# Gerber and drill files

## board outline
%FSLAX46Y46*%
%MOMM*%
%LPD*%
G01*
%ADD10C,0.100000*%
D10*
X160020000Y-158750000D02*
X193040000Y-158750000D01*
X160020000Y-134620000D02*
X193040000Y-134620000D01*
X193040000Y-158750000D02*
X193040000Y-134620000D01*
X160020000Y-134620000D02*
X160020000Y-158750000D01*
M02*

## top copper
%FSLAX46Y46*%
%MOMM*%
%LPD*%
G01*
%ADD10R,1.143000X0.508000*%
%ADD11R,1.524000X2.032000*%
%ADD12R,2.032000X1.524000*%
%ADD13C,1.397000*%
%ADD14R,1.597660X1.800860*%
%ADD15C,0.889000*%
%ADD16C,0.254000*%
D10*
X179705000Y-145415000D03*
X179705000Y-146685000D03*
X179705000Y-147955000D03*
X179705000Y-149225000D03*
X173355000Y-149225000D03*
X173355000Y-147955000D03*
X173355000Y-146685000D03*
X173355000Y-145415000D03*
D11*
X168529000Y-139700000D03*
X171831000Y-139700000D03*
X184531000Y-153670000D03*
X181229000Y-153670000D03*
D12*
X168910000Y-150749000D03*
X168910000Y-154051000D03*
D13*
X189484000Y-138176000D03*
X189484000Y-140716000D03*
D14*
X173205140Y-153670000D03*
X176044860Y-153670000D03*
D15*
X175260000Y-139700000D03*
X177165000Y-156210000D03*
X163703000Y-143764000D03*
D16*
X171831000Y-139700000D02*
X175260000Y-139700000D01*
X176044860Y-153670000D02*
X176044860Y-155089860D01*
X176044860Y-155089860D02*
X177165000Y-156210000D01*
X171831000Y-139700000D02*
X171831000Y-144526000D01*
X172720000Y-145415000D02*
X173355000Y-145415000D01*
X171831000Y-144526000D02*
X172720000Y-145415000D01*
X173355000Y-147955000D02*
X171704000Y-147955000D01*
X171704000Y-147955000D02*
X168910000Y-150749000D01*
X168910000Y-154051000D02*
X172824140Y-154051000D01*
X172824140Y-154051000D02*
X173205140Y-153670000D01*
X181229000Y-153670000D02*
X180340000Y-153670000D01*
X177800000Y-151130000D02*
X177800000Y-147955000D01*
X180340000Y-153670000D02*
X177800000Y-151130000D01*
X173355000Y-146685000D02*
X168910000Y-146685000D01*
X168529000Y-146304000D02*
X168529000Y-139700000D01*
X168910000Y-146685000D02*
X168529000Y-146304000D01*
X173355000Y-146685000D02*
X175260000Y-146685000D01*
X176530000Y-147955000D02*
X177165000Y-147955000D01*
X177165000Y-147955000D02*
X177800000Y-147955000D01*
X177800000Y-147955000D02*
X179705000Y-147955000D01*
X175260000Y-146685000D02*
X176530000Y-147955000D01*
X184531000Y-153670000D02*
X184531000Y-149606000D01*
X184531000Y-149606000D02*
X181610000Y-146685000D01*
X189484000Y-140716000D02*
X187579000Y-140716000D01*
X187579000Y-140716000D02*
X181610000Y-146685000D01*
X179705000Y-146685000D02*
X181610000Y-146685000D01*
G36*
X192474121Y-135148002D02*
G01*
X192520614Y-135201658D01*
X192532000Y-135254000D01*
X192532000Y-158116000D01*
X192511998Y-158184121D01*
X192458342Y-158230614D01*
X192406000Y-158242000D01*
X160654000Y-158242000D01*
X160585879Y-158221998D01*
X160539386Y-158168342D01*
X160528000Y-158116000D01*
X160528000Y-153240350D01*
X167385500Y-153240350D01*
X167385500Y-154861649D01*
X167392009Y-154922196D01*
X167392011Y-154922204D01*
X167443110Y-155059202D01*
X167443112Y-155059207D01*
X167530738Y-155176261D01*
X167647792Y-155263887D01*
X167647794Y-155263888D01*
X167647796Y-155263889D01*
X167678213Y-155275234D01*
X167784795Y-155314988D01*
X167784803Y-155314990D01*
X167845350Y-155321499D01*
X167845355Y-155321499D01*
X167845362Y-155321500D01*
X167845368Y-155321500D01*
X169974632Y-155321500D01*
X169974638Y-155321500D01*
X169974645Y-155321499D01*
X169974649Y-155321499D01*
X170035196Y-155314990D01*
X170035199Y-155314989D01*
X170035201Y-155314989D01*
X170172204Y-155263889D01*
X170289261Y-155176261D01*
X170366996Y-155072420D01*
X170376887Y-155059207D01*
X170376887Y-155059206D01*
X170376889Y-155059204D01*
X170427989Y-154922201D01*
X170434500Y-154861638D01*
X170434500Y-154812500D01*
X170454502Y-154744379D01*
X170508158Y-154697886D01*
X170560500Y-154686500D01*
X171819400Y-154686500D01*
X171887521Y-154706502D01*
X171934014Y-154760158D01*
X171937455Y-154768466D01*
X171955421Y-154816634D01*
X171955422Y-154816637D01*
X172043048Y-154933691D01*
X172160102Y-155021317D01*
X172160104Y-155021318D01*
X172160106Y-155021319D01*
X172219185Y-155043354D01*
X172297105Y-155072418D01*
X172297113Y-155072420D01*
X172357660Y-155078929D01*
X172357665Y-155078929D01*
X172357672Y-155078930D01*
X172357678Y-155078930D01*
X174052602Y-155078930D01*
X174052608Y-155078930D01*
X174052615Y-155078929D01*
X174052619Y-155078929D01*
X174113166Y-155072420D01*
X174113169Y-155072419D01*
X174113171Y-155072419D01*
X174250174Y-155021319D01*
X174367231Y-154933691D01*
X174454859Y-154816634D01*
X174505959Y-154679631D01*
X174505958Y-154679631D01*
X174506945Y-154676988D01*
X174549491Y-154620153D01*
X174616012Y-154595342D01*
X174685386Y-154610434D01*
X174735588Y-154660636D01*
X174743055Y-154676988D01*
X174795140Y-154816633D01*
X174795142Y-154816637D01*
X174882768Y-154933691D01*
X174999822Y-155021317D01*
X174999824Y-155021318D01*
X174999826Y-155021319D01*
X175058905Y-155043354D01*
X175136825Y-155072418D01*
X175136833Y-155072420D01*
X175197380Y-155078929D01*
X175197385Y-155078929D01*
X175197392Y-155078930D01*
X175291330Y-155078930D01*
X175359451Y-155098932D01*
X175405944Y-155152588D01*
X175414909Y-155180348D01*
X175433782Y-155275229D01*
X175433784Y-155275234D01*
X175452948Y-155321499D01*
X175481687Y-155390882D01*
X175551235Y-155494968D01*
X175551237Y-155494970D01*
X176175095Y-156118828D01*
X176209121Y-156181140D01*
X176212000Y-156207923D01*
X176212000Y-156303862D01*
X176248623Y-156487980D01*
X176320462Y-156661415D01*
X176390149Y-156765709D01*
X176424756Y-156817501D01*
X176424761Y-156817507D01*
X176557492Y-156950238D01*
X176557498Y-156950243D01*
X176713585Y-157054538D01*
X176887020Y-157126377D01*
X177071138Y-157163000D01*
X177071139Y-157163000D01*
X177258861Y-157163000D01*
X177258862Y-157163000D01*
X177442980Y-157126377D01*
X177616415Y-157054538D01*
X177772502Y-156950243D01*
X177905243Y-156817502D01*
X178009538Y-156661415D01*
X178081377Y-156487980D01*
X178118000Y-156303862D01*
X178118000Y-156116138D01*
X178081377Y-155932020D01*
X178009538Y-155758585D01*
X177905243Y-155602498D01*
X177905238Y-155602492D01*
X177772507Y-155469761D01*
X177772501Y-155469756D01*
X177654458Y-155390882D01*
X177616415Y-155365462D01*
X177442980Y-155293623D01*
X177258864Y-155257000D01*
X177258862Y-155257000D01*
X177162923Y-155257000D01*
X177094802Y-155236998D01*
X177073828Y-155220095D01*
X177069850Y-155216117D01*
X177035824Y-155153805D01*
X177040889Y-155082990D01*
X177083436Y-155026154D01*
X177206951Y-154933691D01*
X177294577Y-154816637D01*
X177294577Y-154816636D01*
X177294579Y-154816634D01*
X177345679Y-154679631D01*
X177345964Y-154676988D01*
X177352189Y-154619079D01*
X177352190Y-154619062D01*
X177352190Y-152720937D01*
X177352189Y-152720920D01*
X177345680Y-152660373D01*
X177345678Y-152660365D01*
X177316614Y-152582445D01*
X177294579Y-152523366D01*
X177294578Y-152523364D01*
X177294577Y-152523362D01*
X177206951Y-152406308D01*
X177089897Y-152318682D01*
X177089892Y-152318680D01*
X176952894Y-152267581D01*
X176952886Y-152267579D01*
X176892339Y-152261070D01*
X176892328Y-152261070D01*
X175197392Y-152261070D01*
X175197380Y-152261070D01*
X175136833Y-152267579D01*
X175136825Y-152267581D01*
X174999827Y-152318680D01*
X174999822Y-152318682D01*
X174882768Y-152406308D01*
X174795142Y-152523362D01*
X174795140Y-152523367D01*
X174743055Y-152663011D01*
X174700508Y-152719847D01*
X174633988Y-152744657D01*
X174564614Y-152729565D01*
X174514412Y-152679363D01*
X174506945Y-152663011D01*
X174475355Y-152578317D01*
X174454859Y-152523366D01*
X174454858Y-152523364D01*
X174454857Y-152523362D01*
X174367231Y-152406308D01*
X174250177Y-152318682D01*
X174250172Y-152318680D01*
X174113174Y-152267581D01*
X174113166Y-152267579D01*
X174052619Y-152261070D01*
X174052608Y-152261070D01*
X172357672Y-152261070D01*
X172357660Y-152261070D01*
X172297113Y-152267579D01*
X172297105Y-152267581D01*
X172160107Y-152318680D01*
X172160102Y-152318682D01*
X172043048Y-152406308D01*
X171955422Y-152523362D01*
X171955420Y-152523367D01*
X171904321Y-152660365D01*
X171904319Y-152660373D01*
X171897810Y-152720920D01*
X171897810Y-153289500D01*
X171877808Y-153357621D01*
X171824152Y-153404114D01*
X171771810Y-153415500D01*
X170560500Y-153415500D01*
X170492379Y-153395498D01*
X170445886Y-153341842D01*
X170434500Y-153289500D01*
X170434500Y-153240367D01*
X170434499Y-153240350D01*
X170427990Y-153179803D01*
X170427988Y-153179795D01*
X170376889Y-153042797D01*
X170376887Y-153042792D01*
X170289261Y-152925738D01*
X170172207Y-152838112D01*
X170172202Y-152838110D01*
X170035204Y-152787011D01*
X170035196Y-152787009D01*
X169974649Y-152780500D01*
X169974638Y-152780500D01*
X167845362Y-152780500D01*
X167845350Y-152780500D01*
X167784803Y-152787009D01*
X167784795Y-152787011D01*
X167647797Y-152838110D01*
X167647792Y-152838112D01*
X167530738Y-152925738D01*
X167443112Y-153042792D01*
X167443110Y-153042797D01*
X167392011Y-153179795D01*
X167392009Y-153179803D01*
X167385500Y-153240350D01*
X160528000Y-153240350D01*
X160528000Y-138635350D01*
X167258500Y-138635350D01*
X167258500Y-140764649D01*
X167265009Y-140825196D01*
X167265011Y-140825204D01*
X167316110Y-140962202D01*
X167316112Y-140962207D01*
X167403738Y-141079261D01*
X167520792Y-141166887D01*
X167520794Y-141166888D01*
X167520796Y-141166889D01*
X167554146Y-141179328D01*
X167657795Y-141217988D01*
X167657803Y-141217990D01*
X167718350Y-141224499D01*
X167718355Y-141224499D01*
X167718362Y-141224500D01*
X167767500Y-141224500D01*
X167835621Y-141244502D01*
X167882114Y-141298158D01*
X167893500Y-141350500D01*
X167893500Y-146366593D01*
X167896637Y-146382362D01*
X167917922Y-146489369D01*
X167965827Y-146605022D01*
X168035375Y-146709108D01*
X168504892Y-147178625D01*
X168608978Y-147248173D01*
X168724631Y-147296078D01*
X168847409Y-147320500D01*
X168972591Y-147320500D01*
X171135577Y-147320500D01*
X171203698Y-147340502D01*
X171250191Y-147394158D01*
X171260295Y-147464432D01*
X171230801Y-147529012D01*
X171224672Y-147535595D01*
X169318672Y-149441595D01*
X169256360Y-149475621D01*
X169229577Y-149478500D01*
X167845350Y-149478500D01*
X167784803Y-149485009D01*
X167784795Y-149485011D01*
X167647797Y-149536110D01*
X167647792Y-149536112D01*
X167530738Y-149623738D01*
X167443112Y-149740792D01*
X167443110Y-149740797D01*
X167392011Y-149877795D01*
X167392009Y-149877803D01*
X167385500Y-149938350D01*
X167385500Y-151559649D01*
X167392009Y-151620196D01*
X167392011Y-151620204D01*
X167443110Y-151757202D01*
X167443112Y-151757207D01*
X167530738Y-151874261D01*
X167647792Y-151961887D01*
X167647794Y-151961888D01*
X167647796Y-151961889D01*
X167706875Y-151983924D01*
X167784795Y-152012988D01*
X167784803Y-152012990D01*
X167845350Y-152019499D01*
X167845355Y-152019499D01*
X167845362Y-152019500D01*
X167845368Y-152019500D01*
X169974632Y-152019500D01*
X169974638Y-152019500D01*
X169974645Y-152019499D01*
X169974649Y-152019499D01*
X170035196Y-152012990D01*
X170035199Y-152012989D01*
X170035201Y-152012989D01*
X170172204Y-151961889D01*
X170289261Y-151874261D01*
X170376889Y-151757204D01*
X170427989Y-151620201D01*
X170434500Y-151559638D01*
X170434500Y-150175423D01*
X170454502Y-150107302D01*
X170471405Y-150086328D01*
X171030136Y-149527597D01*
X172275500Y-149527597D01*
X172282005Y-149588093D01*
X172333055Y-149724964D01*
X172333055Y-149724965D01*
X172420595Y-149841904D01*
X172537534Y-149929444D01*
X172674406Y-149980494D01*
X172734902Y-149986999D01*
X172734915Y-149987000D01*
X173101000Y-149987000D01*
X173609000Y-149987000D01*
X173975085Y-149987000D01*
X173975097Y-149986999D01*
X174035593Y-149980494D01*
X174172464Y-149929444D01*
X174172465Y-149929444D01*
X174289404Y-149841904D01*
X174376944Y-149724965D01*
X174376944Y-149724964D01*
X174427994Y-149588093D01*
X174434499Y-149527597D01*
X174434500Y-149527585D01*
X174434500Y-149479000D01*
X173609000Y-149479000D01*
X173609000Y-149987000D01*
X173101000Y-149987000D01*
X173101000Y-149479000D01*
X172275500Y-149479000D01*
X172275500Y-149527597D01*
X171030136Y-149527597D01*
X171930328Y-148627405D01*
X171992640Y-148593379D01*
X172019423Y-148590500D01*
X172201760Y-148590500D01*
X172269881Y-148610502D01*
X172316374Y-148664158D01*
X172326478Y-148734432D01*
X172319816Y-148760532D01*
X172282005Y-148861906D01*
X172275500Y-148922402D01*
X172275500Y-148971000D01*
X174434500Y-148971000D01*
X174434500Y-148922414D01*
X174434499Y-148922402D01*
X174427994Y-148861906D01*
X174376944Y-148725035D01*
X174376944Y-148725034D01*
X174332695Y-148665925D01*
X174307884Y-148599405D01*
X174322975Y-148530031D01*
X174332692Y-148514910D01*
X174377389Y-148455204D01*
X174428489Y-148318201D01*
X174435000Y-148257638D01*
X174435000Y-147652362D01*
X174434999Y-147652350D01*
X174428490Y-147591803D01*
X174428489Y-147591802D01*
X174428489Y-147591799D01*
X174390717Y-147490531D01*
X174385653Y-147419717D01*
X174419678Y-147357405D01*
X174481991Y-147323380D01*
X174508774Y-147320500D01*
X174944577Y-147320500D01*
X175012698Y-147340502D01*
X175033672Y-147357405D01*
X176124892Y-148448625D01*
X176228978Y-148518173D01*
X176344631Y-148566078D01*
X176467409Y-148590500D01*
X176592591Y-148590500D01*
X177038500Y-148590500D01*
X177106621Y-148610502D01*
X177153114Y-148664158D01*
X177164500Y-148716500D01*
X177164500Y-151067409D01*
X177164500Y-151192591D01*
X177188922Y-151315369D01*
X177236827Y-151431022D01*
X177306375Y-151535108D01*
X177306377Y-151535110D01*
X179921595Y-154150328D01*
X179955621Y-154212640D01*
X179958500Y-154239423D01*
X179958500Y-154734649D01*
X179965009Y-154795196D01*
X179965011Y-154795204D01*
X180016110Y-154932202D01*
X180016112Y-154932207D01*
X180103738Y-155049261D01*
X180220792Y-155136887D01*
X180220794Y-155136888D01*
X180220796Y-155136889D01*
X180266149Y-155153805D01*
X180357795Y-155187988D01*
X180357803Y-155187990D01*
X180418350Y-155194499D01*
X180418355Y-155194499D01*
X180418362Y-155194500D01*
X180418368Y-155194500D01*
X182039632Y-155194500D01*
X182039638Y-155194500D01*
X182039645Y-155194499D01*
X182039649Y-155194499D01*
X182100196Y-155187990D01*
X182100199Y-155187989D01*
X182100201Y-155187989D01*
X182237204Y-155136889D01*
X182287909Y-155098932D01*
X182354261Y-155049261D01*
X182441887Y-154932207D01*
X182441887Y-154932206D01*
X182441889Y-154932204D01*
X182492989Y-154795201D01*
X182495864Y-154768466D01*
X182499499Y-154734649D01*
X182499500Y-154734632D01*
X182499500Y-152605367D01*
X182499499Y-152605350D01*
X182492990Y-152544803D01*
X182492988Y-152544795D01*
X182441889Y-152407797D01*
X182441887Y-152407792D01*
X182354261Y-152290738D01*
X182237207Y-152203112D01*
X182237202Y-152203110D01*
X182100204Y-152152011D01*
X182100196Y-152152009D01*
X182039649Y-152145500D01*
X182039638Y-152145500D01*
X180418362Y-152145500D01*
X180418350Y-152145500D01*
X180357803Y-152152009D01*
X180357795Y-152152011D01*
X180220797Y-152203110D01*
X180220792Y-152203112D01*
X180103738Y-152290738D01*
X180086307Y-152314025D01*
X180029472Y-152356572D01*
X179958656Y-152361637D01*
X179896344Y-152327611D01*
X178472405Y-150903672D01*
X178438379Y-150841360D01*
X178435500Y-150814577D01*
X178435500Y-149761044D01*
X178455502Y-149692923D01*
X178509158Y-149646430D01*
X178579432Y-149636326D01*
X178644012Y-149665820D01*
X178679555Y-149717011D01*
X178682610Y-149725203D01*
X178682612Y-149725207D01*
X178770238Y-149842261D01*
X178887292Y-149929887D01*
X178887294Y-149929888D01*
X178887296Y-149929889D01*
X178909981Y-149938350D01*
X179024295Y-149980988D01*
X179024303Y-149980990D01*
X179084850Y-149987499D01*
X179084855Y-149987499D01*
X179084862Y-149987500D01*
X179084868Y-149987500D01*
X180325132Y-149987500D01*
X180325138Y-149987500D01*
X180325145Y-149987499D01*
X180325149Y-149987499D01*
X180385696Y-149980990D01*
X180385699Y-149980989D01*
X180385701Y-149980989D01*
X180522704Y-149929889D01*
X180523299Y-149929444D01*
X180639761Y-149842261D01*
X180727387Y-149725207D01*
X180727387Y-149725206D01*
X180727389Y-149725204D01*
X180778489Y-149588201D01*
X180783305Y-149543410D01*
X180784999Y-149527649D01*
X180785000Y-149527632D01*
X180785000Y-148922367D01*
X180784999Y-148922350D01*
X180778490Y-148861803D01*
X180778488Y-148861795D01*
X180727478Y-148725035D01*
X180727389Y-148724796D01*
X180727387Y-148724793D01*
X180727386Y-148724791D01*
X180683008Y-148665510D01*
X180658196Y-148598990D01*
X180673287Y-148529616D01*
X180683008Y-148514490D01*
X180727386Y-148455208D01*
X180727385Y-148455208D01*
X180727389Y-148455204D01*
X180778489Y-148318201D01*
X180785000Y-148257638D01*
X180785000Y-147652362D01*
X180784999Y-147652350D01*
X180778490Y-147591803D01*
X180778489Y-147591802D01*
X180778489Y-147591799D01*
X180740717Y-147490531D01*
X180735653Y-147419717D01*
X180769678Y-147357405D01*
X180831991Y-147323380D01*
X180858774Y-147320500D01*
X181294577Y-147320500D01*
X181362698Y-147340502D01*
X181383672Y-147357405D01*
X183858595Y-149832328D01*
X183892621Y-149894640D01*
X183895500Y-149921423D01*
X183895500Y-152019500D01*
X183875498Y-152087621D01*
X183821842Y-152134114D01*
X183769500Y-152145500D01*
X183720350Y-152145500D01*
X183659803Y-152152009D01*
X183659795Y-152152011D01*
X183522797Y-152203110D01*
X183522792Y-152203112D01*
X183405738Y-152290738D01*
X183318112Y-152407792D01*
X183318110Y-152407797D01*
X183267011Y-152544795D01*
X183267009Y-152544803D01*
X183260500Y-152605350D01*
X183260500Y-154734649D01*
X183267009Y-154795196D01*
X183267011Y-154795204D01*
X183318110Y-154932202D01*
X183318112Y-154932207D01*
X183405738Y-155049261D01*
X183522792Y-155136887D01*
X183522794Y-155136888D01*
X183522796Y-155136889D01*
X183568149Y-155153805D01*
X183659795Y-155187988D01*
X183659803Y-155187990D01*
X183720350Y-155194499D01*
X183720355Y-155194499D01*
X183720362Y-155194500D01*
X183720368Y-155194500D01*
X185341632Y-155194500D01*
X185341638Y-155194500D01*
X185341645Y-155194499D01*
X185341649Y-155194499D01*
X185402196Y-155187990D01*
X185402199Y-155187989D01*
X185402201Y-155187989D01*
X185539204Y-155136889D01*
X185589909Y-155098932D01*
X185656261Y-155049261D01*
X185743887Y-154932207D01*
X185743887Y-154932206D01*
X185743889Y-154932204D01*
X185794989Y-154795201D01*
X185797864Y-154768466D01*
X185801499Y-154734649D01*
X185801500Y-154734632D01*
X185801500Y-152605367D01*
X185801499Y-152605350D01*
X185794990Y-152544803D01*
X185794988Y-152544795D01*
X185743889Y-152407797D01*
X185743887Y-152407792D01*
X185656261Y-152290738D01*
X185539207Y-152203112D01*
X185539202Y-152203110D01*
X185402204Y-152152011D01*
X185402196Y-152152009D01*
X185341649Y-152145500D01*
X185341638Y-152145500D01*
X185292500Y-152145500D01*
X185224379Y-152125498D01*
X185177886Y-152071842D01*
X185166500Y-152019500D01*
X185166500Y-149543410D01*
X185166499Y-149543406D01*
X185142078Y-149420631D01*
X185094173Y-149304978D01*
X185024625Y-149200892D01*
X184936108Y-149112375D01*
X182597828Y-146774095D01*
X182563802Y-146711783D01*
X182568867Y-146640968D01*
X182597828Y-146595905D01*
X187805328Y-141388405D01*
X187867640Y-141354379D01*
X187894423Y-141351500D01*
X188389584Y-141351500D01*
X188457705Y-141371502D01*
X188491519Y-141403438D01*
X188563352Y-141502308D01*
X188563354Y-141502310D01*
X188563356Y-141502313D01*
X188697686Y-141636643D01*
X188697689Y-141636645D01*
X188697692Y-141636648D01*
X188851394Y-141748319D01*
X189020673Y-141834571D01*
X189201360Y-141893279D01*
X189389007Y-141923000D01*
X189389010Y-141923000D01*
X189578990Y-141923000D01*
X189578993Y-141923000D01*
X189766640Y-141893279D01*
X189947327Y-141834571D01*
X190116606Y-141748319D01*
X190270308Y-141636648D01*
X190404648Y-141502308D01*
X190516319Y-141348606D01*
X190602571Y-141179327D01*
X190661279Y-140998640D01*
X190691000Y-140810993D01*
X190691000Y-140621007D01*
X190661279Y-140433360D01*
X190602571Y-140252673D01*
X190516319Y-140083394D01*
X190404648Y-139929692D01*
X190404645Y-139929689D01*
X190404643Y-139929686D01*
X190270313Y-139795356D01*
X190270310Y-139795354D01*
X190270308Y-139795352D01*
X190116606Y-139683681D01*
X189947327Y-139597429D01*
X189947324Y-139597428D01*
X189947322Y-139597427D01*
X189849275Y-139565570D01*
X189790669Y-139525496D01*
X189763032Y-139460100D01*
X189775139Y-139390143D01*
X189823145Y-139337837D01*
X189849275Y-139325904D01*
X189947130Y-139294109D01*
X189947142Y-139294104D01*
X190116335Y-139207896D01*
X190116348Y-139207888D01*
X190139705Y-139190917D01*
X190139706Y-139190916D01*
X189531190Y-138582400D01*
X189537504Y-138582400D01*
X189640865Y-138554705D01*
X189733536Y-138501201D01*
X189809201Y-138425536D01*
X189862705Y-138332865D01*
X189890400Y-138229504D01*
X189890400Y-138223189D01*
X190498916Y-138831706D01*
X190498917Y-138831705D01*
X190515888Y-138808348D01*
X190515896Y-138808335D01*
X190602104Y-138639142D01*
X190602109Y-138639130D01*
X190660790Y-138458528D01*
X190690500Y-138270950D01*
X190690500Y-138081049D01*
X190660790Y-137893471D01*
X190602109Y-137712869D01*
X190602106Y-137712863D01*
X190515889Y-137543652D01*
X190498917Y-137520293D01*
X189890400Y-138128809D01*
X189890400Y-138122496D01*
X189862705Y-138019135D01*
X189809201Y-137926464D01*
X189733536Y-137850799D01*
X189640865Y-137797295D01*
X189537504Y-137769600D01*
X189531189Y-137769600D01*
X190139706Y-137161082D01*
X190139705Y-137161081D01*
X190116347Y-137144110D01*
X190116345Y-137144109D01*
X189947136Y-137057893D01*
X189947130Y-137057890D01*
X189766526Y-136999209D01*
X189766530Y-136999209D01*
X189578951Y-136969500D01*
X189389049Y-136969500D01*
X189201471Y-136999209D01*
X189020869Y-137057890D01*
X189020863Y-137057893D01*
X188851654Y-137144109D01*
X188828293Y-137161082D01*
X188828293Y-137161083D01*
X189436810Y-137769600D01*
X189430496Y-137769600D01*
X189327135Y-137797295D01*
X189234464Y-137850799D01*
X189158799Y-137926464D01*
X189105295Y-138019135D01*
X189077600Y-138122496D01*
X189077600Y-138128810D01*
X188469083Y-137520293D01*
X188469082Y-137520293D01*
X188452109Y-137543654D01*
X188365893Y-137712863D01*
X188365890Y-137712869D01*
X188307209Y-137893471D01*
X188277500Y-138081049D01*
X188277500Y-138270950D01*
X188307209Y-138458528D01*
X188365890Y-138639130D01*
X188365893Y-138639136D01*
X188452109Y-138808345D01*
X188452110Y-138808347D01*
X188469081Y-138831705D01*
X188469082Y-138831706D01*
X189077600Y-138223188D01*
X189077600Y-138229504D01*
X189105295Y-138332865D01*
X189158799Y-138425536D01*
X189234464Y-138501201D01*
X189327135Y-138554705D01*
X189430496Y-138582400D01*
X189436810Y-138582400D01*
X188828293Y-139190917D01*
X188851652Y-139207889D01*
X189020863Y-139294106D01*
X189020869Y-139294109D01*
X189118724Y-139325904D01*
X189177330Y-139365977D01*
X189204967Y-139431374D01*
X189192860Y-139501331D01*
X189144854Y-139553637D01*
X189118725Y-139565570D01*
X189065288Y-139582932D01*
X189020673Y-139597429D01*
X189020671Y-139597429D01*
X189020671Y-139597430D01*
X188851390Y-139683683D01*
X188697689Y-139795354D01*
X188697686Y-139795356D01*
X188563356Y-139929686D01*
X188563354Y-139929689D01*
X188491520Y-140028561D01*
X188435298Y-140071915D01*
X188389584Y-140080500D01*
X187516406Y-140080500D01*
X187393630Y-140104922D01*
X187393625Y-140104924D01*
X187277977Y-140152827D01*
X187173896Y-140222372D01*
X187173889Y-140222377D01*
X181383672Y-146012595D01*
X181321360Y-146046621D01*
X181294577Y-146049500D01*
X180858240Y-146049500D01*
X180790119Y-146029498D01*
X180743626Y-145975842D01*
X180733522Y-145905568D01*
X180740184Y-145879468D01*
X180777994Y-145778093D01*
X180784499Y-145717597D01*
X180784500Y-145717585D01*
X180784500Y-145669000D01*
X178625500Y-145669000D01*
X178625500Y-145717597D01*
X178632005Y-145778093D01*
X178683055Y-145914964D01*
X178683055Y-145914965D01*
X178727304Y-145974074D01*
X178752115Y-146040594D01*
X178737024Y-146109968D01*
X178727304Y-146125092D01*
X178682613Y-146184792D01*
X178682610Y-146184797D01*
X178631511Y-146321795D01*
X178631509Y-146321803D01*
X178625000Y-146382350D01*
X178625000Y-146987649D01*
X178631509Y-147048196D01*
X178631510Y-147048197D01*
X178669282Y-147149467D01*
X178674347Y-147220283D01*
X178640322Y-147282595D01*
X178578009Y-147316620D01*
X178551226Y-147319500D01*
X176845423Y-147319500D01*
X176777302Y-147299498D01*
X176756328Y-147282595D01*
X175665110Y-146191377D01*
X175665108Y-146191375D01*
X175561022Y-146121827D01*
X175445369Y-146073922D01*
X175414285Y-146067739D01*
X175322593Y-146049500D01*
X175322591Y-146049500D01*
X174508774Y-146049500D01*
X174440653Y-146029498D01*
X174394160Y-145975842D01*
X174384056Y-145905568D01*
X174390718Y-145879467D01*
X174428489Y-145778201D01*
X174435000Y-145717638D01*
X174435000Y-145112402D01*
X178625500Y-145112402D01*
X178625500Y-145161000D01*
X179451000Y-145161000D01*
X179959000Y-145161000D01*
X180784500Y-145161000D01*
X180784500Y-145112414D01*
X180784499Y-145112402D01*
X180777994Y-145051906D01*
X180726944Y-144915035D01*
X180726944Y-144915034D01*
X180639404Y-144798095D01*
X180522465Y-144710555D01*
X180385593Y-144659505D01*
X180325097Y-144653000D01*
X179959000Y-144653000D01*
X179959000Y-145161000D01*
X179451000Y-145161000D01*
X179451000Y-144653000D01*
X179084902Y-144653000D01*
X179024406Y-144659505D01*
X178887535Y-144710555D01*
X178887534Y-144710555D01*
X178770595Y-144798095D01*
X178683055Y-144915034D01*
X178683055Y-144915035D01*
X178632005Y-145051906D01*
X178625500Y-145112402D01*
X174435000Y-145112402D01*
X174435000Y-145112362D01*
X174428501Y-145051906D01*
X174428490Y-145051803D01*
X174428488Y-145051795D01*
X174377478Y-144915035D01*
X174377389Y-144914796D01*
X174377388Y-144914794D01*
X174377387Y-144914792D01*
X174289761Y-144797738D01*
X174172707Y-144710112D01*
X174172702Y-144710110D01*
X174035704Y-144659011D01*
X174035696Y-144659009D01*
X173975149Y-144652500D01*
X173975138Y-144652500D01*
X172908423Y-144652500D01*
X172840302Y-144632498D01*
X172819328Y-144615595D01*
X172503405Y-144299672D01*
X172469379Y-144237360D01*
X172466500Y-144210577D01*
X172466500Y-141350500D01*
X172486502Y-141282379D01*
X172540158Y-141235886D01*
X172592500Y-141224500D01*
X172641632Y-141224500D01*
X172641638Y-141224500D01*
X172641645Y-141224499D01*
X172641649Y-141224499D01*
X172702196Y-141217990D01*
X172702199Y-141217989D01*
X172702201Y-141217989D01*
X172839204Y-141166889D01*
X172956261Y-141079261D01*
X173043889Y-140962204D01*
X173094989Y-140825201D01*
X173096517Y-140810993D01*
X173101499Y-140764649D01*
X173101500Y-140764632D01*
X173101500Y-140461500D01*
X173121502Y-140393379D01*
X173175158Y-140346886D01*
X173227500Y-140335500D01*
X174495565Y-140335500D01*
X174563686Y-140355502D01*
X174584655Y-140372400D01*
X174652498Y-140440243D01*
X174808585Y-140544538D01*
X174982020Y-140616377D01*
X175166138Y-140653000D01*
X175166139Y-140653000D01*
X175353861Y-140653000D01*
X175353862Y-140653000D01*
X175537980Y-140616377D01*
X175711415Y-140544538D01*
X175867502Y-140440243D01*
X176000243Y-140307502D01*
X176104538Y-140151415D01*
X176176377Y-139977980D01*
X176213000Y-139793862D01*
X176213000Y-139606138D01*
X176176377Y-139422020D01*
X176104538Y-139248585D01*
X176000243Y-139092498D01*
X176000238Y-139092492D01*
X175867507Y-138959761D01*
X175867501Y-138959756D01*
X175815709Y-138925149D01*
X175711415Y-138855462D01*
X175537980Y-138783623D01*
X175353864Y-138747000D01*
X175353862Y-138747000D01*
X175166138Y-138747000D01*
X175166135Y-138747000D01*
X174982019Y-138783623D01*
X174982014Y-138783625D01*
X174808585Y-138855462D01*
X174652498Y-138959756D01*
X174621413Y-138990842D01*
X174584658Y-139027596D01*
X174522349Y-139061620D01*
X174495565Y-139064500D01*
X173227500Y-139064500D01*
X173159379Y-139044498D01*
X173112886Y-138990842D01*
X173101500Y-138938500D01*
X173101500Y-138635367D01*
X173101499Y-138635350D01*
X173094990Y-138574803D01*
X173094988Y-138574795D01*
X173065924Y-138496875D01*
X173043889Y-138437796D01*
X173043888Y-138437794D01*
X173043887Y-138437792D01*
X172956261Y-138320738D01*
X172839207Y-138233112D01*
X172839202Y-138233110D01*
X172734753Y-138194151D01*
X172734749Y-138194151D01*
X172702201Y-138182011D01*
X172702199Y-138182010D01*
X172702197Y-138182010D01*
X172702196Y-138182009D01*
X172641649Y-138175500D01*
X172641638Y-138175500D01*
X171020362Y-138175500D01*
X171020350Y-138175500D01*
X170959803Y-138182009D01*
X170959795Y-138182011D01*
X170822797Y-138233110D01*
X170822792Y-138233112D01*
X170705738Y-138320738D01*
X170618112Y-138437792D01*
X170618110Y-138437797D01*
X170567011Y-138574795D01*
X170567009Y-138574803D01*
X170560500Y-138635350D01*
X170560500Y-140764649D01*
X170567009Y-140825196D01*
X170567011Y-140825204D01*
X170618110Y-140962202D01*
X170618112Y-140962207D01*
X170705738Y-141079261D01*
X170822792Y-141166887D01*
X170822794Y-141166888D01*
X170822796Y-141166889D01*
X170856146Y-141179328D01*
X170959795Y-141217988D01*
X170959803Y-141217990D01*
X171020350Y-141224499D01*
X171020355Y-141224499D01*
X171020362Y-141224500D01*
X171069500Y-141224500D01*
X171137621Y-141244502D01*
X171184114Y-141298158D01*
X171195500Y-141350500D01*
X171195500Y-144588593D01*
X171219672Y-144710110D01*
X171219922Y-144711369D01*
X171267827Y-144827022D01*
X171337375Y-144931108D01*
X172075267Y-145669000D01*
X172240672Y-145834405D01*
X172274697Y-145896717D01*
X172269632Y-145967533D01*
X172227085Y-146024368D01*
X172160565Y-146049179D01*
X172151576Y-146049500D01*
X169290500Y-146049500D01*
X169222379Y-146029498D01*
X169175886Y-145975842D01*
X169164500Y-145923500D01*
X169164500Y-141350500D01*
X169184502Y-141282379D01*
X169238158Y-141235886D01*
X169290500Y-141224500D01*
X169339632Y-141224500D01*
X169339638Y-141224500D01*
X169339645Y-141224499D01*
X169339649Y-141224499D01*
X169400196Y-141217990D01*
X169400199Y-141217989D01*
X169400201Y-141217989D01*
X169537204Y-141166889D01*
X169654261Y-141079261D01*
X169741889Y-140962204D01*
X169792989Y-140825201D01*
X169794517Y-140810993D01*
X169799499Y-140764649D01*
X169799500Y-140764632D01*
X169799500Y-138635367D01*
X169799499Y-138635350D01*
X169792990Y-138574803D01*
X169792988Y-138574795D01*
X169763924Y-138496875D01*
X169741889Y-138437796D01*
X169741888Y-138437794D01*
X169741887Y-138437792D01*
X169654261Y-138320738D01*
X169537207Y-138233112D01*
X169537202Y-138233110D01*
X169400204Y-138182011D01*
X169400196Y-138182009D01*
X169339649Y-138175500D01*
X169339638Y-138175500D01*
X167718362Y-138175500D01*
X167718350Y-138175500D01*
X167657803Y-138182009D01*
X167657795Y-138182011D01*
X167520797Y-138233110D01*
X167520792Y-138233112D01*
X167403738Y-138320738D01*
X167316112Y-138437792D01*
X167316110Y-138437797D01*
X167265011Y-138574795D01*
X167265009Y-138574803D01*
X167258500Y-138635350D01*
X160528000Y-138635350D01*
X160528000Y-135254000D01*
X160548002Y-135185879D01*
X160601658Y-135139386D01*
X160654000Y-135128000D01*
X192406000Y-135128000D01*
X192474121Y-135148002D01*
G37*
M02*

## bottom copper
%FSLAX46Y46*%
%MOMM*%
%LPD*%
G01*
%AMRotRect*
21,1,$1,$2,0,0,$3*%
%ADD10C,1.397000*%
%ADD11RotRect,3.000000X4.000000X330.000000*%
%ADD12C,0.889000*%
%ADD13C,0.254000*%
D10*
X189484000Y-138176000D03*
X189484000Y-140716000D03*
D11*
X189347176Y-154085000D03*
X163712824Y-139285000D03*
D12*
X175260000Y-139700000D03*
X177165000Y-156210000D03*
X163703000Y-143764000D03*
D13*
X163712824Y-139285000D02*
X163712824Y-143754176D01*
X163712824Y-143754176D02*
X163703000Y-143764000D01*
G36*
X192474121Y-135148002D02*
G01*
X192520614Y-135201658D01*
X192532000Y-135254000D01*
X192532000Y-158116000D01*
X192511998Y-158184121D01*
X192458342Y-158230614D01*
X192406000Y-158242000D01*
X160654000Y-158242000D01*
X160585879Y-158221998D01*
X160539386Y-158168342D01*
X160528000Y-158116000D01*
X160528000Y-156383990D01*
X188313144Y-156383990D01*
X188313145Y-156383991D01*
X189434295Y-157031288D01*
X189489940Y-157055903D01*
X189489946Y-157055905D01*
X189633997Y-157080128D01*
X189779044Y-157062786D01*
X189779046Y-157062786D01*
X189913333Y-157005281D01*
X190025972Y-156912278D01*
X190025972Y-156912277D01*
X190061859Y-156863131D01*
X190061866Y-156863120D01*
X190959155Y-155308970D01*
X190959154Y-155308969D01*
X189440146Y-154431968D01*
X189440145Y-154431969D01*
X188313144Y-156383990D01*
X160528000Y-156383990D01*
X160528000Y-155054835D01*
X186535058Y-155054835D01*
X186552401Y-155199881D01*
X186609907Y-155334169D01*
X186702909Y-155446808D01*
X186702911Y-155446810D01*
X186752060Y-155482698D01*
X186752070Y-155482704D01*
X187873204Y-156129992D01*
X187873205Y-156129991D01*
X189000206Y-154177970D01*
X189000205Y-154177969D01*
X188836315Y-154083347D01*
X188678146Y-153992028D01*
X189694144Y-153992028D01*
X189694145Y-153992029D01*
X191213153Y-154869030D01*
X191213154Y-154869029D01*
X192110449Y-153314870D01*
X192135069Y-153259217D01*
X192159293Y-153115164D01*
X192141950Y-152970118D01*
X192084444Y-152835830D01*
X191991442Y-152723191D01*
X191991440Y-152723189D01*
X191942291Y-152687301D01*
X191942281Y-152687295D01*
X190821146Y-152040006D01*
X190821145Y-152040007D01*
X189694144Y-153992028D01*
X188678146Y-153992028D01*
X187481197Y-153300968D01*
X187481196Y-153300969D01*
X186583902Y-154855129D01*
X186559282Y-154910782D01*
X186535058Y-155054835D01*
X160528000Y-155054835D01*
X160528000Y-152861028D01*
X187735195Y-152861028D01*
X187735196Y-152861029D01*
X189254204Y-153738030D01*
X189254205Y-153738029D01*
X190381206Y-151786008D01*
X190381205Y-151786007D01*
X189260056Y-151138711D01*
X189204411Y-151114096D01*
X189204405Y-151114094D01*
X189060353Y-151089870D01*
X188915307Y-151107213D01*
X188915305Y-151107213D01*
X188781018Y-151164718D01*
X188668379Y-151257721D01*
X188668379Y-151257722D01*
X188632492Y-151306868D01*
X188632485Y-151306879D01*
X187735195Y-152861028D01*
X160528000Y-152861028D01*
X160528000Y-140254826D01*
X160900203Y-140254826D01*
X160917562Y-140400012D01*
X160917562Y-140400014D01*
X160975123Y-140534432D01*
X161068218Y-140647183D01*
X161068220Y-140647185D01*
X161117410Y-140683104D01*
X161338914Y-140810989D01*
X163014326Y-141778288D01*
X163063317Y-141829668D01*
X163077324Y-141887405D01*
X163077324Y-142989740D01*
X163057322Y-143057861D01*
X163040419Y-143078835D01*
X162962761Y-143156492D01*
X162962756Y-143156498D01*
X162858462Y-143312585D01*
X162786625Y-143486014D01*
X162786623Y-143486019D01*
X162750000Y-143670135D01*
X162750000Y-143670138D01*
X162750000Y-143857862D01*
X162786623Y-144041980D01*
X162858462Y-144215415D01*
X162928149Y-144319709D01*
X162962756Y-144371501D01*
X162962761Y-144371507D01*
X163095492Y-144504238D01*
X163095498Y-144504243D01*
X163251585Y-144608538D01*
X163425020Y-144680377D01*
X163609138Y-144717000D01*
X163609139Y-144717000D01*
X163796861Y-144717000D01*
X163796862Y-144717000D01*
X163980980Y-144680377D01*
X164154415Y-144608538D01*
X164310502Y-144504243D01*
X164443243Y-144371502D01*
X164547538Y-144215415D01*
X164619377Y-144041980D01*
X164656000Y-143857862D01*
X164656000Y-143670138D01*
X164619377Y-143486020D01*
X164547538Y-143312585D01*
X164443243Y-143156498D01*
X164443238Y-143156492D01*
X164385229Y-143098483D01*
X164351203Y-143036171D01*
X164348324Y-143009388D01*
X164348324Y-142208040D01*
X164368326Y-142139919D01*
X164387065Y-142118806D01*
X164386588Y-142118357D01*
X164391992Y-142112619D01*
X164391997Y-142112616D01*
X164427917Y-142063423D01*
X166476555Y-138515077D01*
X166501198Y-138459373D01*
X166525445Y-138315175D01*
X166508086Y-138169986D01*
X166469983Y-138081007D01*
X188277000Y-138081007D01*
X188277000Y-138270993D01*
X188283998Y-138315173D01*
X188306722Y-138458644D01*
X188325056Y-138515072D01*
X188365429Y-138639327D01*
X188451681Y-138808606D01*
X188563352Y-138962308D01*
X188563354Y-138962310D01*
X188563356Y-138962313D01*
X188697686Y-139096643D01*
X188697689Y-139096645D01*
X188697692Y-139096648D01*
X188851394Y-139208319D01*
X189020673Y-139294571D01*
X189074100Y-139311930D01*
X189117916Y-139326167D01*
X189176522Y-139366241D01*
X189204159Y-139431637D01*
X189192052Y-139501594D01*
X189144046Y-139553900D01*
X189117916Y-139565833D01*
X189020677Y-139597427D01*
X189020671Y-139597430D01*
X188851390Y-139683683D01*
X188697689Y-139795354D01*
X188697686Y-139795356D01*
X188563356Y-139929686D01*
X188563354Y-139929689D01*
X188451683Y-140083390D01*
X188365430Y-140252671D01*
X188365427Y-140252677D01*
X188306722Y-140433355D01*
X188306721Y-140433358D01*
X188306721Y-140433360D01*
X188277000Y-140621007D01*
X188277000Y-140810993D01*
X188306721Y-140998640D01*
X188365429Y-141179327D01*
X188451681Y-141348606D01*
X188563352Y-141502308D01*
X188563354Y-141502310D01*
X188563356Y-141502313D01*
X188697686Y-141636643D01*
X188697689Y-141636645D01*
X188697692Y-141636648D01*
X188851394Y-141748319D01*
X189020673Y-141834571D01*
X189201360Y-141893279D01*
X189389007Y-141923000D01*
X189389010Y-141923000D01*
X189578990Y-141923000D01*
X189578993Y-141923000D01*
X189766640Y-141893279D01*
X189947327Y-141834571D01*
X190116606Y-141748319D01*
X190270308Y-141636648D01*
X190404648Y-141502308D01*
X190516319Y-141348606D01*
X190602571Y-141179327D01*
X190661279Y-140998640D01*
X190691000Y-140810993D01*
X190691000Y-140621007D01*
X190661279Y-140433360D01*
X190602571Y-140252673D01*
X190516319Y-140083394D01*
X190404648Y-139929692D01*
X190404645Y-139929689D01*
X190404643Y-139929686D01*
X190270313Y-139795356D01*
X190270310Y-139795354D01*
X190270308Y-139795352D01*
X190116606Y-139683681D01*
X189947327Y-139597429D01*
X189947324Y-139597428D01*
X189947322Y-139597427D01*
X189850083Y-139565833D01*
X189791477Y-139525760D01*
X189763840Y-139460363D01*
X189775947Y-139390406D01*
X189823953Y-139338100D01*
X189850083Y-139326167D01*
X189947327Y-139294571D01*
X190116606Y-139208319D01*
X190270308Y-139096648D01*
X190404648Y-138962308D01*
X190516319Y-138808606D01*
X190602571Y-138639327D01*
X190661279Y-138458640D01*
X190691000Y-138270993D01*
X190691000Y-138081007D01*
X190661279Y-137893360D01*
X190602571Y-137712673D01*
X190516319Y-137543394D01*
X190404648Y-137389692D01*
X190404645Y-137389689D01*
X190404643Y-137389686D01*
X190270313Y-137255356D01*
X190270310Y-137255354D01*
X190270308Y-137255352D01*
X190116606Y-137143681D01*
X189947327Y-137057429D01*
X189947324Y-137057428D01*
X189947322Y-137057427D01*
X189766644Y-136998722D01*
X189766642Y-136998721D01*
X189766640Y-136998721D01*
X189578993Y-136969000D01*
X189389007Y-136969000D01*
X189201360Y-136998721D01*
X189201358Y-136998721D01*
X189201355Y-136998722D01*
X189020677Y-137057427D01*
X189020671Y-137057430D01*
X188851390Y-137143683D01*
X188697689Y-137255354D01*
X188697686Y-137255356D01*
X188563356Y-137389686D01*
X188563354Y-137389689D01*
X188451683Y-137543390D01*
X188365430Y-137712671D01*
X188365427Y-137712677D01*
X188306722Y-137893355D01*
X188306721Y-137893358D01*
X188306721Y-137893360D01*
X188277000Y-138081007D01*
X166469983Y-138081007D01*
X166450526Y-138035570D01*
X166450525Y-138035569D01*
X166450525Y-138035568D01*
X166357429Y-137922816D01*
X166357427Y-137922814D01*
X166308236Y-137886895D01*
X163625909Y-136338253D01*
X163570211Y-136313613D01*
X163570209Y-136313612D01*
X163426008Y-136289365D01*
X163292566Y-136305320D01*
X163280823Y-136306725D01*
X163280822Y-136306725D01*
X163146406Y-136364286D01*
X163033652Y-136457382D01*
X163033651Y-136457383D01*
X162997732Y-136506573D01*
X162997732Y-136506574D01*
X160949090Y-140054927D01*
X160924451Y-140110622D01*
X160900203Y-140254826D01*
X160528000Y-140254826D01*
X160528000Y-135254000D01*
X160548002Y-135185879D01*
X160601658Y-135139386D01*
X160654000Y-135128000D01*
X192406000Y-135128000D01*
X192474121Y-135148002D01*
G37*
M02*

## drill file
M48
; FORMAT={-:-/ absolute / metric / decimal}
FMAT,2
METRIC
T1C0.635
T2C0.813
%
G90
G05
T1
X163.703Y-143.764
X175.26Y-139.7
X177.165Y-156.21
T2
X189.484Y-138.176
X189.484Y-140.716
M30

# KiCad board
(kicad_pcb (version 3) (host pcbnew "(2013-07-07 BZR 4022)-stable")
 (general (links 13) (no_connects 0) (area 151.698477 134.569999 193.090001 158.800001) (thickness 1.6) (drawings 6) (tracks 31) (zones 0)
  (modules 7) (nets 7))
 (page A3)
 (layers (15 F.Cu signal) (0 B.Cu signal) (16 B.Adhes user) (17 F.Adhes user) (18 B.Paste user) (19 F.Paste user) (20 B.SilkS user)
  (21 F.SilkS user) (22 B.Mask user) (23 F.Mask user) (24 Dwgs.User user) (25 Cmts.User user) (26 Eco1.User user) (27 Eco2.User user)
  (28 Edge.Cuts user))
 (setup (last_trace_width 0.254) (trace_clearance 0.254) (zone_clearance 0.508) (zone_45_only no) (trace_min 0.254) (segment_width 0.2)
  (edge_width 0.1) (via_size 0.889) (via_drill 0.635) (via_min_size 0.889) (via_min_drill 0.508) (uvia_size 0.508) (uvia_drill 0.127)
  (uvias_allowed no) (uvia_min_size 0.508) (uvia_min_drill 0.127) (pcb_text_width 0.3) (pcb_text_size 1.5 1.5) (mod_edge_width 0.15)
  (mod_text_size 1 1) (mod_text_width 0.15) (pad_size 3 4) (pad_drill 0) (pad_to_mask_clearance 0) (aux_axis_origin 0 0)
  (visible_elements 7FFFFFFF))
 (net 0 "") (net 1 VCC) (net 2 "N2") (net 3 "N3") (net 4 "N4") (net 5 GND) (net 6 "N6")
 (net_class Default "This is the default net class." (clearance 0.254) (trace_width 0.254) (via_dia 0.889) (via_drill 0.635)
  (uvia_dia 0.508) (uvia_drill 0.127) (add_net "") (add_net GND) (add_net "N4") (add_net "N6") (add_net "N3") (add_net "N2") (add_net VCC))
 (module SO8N (layer F.Cu) (at 176.53 147.32 270)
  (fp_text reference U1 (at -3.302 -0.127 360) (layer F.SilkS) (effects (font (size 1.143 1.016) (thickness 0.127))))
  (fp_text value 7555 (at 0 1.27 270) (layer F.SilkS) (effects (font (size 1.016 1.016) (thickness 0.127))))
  (pad 8 smd rect (at -1.905 -3.175 270) (size 0.508 1.143) (layers F.Cu F.Paste F.Mask) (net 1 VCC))
  (pad 7 smd rect (at -0.635 -3.175 270) (size 0.508 1.143) (layers F.Cu F.Paste F.Mask) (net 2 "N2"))
  (pad 6 smd rect (at 0.635 -3.175 270) (size 0.508 1.143) (layers F.Cu F.Paste F.Mask) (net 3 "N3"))
  (pad 5 smd rect (at 1.905 -3.175 270) (size 0.508 1.143) (layers F.Cu F.Paste F.Mask))
  (pad 4 smd rect (at 1.905 3.175 270) (size 0.508 1.143) (layers F.Cu F.Paste F.Mask) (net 1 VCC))
  (pad 3 smd rect (at 0.635 3.175 270) (size 0.508 1.143) (layers F.Cu F.Paste F.Mask) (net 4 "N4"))
  (pad 2 smd rect (at -0.635 3.175 270) (size 0.508 1.143) (layers F.Cu F.Paste F.Mask) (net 3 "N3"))
  (pad 1 smd rect (at -1.905 3.175 270) (size 0.508 1.143) (layers F.Cu F.Paste F.Mask) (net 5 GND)))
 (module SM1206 (layer F.Cu) (at 170.18 139.7)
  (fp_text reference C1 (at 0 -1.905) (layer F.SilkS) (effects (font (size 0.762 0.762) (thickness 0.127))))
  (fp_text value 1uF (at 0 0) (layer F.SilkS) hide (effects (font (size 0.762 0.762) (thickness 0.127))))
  (pad 1 smd rect (at -1.651 0) (size 1.524 2.032) (layers F.Cu F.Paste F.Mask) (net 3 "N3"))
  (pad 2 smd rect (at 1.651 0) (size 1.524 2.032) (layers F.Cu F.Paste F.Mask) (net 5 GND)))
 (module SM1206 (layer F.Cu) (at 182.88 153.67 180)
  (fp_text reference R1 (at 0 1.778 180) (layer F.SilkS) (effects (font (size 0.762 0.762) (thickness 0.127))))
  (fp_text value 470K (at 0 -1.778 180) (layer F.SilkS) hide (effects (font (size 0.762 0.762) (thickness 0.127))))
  (pad 1 smd rect (at -1.651 0 180) (size 1.524 2.032) (layers F.Cu F.Paste F.Mask) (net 2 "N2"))
  (pad 2 smd rect (at 1.651 0 180) (size 1.524 2.032) (layers F.Cu F.Paste F.Mask) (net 3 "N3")))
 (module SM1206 (layer F.Cu) (at 168.91 152.4 270)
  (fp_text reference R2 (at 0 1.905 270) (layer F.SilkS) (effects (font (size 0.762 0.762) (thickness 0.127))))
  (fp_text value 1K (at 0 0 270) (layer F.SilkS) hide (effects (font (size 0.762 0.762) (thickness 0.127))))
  (pad 1 smd rect (at -1.651 0 270) (size 1.524 2.032) (layers F.Cu F.Paste F.Mask) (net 4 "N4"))
  (pad 2 smd rect (at 1.651 0 270) (size 1.524 2.032) (layers F.Cu F.Paste F.Mask) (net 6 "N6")))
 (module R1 (layer F.Cu) (at 189.484 139.446 270) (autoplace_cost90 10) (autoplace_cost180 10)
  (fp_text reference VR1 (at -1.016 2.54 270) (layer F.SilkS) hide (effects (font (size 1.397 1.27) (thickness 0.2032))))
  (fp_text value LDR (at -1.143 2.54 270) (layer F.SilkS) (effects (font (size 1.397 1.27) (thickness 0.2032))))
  (pad 1 thru_hole circle (at -1.27 0 270) (size 1.397 1.397) (drill 0.8128) (layers *.Cu *.Mask F.SilkS) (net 1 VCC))
  (pad 2 thru_hole circle (at 1.27 0 270) (size 1.397 1.397) (drill 0.8128) (layers *.Cu *.Mask F.SilkS) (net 2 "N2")))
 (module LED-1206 (layer F.Cu) (at 174.625 153.67)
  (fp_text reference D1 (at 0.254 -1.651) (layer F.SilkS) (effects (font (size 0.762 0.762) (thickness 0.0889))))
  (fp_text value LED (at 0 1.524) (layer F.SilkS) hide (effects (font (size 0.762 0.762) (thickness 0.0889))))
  (pad 1 smd rect (at -1.41986 0) (size 1.59766 1.80086) (layers F.Cu F.Paste F.Mask) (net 6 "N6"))
  (pad 2 smd rect (at 1.41986 0) (size 1.59766 1.80086) (layers F.Cu F.Paste F.Mask) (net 5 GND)))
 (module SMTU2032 (layer B.Cu) (at 176.53 146.685 330)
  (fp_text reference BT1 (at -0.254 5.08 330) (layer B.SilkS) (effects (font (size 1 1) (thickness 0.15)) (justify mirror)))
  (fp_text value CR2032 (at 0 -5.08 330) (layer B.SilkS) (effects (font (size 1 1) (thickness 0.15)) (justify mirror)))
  (pad 2 smd rect (at 14.8 0 330) (size 3 4) (layers B.Cu B.Paste B.Mask) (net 5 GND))
  (pad 1 smd rect (at -14.8 0 330) (size 3 4) (layers B.Cu B.Paste B.Mask) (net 1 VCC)))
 (gr_line (start 160.02 158.75) (end 193.04 158.75) (angle 90) (layer Edge.Cuts) (width 0.1))
 (gr_line (start 160.02 134.62) (end 193.04 134.62) (angle 90) (layer Edge.Cuts) (width 0.1))
 (gr_line (start 193.04 158.75) (end 193.04 134.62) (angle 90) (layer Edge.Cuts) (width 0.1))
 (gr_line (start 160.02 134.62) (end 160.02 158.75) (angle 90) (layer Edge.Cuts) (width 0.1))
 (segment (start 171.831 139.7) (end 175.26 139.7) (width 0.254) (layer F.Cu) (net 5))
 (via (at 175.26 139.7) (size 0.889) (layers F.Cu B.Cu) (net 5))
 (segment (start 176.04486 153.67) (end 176.04486 155.08986) (width 0.254) (layer F.Cu) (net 5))
 (via (at 177.165 156.21) (size 0.889) (layers F.Cu B.Cu) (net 5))
 (segment (start 176.04486 155.08986) (end 177.165 156.21) (width 0.254) (layer F.Cu) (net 5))
 (segment (start 171.831 139.7) (end 171.831 144.526) (width 0.254) (layer F.Cu) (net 5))
 (segment (start 172.72 145.415) (end 173.355 145.415) (width 0.254) (layer F.Cu) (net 5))
 (segment (start 171.831 144.526) (end 172.72 145.415) (width 0.254) (layer F.Cu) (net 5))
 (segment (start 173.355 147.955) (end 171.704 147.955) (width 0.254) (layer F.Cu) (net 4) (status 10))
 (segment (start 171.704 147.955) (end 168.91 150.749) (width 0.254) (layer F.Cu) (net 4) (status 20))
 (segment (start 168.91 154.051) (end 172.82414 154.051) (width 0.254) (layer F.Cu) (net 6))
 (segment (start 172.82414 154.051) (end 173.20514 153.67) (width 0.254) (layer F.Cu) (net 6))
 (segment (start 181.229 153.67) (end 180.34 153.67) (width 0.254) (layer F.Cu) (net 3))
 (segment (start 177.8 151.13) (end 177.8 147.955) (width 0.254) (layer F.Cu) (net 3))
 (segment (start 180.34 153.67) (end 177.8 151.13) (width 0.254) (layer F.Cu) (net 3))
 (segment (start 173.355 146.685) (end 168.91 146.685) (width 0.254) (layer F.Cu) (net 3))
 (segment (start 168.529 146.304) (end 168.529 139.7) (width 0.254) (layer F.Cu) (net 3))
 (segment (start 168.91 146.685) (end 168.529 146.304) (width 0.254) (layer F.Cu) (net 3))
 (segment (start 173.355 146.685) (end 175.26 146.685) (width 0.254) (layer F.Cu) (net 3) (status 10))
 (segment (start 176.53 147.955) (end 177.165 147.955) (width 0.254) (layer F.Cu) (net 3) (status 20))
 (segment (start 177.165 147.955) (end 177.8 147.955) (width 0.254) (layer F.Cu) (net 3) (status 20))
 (segment (start 177.8 147.955) (end 179.705 147.955) (width 0.254) (layer F.Cu) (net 3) (status 20))
 (segment (start 175.26 146.685) (end 176.53 147.955) (width 0.254) (layer F.Cu) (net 3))
 (segment (start 184.531 153.67) (end 184.531 149.606) (width 0.254) (layer F.Cu) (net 2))
 (segment (start 184.531 149.606) (end 181.61 146.685) (width 0.254) (layer F.Cu) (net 2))
 (segment (start 189.484 140.716) (end 187.579 140.716) (width 0.254) (layer F.Cu) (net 2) (status 10))
 (segment (start 187.579 140.716) (end 181.61 146.685) (width 0.254) (layer F.Cu) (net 2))
 (segment (start 179.705 146.685) (end 181.61 146.685) (width 0.254) (layer F.Cu) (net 2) (status 10))
 (segment (start 163.712824 139.285) (end 163.712824 143.754176) (width 0.254) (layer B.Cu) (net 1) (status 10))
 (via (at 163.703 143.764) (size 0.889) (layers F.Cu B.Cu) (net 1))
 (segment (start 163.712824 143.754176) (end 163.703 143.764) (width 0.254) (layer B.Cu) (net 1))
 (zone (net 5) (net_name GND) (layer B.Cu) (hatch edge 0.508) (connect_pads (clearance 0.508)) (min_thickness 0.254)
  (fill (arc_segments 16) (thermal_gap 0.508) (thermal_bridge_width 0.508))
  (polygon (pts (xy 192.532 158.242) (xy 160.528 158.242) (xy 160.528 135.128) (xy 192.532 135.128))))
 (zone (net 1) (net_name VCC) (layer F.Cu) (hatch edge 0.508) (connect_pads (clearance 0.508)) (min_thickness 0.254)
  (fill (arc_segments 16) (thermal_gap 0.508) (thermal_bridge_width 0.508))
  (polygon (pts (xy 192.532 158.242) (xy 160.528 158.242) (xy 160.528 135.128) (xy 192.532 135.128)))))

